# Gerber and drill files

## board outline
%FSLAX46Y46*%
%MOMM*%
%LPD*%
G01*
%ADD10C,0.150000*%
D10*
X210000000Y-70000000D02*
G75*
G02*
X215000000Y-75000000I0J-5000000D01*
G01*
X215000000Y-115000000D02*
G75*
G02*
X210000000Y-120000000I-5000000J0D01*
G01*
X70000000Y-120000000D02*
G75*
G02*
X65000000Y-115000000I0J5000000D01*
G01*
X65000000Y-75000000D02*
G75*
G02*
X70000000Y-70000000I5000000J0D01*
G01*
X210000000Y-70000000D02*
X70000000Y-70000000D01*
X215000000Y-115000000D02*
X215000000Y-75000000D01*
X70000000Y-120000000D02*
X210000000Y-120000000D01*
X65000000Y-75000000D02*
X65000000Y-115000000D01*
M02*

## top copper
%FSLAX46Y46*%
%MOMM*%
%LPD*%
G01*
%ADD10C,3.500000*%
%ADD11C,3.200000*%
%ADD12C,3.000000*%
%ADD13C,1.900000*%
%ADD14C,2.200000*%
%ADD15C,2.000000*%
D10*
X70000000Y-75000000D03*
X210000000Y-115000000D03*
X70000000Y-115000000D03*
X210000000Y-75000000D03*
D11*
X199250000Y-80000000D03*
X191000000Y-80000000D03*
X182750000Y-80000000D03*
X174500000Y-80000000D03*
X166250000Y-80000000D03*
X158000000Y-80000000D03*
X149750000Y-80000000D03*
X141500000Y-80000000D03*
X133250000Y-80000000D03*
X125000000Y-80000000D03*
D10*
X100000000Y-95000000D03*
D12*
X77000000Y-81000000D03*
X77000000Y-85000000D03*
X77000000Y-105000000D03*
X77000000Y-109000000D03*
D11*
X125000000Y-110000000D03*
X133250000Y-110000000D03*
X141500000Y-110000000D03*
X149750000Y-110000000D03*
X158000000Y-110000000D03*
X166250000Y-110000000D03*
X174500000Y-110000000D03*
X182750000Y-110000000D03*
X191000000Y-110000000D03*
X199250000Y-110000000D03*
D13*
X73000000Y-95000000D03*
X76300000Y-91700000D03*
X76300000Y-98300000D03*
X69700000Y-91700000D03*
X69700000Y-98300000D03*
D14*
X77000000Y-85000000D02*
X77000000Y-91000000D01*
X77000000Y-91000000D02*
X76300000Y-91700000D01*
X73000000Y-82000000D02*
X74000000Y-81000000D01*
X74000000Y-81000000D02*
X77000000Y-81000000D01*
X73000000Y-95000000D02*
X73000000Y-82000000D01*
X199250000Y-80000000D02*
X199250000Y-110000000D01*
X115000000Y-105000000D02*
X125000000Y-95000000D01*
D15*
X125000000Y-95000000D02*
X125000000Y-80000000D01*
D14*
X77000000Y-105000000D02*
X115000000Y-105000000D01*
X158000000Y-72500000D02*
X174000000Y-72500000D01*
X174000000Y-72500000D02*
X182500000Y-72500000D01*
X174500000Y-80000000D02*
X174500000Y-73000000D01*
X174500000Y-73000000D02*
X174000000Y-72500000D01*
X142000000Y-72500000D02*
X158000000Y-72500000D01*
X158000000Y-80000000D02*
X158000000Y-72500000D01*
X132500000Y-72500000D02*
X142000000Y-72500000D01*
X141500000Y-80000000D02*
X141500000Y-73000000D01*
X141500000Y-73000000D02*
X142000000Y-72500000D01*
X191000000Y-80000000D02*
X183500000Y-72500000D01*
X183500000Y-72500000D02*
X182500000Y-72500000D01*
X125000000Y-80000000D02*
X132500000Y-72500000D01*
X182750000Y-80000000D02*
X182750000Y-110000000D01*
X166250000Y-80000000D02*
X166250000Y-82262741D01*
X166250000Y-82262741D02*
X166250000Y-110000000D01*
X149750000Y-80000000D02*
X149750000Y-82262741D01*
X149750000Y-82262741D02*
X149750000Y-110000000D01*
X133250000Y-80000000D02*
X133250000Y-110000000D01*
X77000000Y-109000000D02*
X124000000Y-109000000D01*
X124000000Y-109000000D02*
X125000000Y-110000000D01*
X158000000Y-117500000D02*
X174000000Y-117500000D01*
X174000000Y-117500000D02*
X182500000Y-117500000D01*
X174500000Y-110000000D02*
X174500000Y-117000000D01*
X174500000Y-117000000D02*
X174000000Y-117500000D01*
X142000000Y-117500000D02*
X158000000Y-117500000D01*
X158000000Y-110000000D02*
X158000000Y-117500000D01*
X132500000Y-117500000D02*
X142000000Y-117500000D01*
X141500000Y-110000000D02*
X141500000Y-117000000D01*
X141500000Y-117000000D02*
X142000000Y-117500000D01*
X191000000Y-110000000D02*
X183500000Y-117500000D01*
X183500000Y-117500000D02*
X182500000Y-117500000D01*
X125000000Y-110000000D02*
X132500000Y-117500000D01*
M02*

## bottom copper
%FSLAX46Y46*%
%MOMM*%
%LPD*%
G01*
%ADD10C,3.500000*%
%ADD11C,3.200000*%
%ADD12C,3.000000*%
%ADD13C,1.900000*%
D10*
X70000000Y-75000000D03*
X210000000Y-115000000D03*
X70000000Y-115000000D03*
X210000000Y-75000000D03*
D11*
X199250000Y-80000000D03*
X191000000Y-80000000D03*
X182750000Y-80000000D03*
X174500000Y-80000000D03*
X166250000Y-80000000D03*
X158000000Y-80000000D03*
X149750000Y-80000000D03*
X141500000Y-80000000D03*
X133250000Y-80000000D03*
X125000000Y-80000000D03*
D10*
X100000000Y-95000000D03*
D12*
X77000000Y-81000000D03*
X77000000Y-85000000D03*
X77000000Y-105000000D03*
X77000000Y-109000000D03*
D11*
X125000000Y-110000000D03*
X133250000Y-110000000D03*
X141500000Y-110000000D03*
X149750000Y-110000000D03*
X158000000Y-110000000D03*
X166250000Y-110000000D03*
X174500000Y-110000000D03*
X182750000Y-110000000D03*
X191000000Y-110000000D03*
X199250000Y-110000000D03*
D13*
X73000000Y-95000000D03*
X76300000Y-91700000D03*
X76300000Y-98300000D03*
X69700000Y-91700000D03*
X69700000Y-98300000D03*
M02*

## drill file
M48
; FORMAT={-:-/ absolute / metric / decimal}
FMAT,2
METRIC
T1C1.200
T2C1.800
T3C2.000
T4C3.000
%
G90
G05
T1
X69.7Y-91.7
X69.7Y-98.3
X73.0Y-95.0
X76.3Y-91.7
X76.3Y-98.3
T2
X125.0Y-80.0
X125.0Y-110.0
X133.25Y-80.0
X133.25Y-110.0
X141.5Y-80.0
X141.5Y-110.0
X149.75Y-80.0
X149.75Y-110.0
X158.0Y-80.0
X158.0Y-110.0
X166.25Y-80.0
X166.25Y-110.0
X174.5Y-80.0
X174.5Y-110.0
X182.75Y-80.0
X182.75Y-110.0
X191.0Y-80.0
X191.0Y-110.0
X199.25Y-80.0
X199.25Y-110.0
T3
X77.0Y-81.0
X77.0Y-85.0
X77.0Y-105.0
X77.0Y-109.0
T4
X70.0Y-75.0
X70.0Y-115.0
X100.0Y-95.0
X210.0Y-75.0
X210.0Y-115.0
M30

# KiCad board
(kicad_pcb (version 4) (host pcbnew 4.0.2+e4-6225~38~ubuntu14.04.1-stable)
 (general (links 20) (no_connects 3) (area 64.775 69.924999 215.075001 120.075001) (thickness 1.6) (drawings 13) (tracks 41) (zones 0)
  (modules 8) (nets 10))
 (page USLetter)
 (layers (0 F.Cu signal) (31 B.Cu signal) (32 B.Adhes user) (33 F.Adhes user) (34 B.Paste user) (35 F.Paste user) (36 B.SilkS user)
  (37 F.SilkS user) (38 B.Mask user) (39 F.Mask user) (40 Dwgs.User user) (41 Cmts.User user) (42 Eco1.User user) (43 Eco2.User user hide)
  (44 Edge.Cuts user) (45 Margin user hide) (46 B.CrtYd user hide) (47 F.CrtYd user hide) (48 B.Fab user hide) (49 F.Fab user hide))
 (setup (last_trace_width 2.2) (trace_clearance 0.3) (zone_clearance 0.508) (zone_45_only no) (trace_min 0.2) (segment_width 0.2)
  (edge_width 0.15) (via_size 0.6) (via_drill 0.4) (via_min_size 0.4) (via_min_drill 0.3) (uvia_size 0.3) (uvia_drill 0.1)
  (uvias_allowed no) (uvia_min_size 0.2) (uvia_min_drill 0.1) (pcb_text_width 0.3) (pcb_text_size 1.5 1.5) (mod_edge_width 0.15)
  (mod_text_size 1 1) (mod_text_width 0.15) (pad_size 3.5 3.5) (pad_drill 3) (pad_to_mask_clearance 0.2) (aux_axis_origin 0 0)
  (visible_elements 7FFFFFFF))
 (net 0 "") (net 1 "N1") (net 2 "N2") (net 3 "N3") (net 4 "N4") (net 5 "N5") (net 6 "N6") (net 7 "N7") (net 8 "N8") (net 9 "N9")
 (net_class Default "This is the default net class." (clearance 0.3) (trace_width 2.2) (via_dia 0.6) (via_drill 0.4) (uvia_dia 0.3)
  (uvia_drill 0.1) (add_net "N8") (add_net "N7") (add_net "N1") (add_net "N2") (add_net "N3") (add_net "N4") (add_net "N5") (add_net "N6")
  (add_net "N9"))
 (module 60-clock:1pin (layer F.Cu) (at 70 75)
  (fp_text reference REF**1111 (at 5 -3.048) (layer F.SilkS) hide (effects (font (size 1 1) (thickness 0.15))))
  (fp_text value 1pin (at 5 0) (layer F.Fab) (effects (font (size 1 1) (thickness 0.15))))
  (pad 1 thru_hole circle (at 0 0) (size 3.5 3.5) (drill 3) (layers *.Cu *.Mask)))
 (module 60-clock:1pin (layer F.Cu) (at 210 115)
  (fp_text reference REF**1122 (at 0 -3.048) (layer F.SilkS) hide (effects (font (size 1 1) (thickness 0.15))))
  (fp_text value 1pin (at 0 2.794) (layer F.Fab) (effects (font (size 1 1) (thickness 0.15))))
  (pad 1 thru_hole circle (at 0 0) (size 3.5 3.5) (drill 3) (layers *.Cu *.Mask)))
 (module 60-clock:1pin (layer F.Cu) (at 70 115)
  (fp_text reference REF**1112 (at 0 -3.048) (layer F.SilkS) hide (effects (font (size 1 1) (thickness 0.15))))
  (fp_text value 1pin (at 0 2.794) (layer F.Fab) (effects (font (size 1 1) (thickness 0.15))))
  (pad 1 thru_hole circle (at 0 0) (size 3.5 3.5) (drill 3) (layers *.Cu *.Mask)))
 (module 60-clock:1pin (layer F.Cu) (at 210 75)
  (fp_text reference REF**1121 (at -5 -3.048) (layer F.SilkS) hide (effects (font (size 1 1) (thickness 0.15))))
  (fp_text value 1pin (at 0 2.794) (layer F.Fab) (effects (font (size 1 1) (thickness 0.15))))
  (pad 1 thru_hole circle (at 0 0) (size 3.5 3.5) (drill 3) (layers *.Cu *.Mask)))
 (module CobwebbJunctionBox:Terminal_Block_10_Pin (layer F.Cu) (at 199.25 80 180)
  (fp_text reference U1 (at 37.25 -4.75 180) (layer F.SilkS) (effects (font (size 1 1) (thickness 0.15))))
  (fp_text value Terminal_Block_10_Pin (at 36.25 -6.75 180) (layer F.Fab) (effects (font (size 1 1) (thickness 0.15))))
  (pad 1 thru_hole circle (at 0 0 180) (size 3.2 3.2) (drill 1.8) (layers *.Cu *.Mask F.SilkS) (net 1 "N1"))
  (pad 2 thru_hole circle (at 8.25 0 180) (size 3.2 3.2) (drill 1.8) (layers *.Cu *.Mask F.SilkS) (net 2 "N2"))
  (pad 3 thru_hole circle (at 16.5 0 180) (size 3.2 3.2) (drill 1.8) (layers *.Cu *.Mask F.SilkS) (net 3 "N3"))
  (pad 4 thru_hole circle (at 24.75 0 180) (size 3.2 3.2) (drill 1.8) (layers *.Cu *.Mask F.SilkS) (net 2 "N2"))
  (pad 5 thru_hole circle (at 33 0 180) (size 3.2 3.2) (drill 1.8) (layers *.Cu *.Mask F.SilkS) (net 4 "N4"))
  (pad 6 thru_hole circle (at 41.25 0 180) (size 3.2 3.2) (drill 1.8) (layers *.Cu *.Mask F.SilkS) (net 2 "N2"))
  (pad 7 thru_hole circle (at 49.5 0 180) (size 3.2 3.2) (drill 1.8) (layers *.Cu *.Mask F.SilkS) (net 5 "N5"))
  (pad 8 thru_hole circle (at 57.75 0 180) (size 3.2 3.2) (drill 1.8) (layers *.Cu *.Mask F.SilkS) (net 2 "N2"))
  (pad 9 thru_hole circle (at 66 0 180) (size 3.2 3.2) (drill 1.8) (layers *.Cu *.Mask F.SilkS) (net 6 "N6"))
  (pad 10 thru_hole circle (at 74.25 0 180) (size 3.2 3.2) (drill 1.8) (layers *.Cu *.Mask F.SilkS) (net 2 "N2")))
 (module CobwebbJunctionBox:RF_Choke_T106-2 (layer F.Cu) (at 100 95)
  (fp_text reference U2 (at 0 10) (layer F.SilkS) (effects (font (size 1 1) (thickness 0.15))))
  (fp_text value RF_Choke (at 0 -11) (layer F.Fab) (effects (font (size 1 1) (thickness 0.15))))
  (pad "" thru_hole circle (at 0 0) (size 3.5 3.5) (drill 3) (layers *.Cu *.Mask F.SilkS))
  (pad 1 thru_hole circle (at -23 -14) (size 3 3) (drill 2) (layers *.Cu *.Mask F.SilkS) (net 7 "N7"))
  (pad 2 thru_hole circle (at -23 -10) (size 3 3) (drill 2) (layers *.Cu *.Mask F.SilkS) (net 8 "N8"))
  (pad 3 thru_hole circle (at -23 10) (size 3 3) (drill 2) (layers *.Cu *.Mask F.SilkS) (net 2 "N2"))
  (pad 4 thru_hole circle (at -23 14) (size 3 3) (drill 2) (layers *.Cu *.Mask F.SilkS) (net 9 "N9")))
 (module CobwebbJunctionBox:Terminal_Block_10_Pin (layer F.Cu) (at 125 110)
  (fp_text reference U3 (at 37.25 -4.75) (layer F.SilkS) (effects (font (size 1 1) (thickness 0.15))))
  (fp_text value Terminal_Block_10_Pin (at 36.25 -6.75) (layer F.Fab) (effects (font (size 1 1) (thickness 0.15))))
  (pad 1 thru_hole circle (at 0 0) (size 3.2 3.2) (drill 1.8) (layers *.Cu *.Mask F.SilkS) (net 9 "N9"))
  (pad 2 thru_hole circle (at 8.25 0) (size 3.2 3.2) (drill 1.8) (layers *.Cu *.Mask F.SilkS) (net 6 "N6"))
  (pad 3 thru_hole circle (at 16.5 0) (size 3.2 3.2) (drill 1.8) (layers *.Cu *.Mask F.SilkS) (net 9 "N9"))
  (pad 4 thru_hole circle (at 24.75 0) (size 3.2 3.2) (drill 1.8) (layers *.Cu *.Mask F.SilkS) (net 5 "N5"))
  (pad 5 thru_hole circle (at 33 0) (size 3.2 3.2) (drill 1.8) (layers *.Cu *.Mask F.SilkS) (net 9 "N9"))
  (pad 6 thru_hole circle (at 41.25 0) (size 3.2 3.2) (drill 1.8) (layers *.Cu *.Mask F.SilkS) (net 4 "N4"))
  (pad 7 thru_hole circle (at 49.5 0) (size 3.2 3.2) (drill 1.8) (layers *.Cu *.Mask F.SilkS) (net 9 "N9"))
  (pad 8 thru_hole circle (at 57.75 0) (size 3.2 3.2) (drill 1.8) (layers *.Cu *.Mask F.SilkS) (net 3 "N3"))
  (pad 9 thru_hole circle (at 66 0) (size 3.2 3.2) (drill 1.8) (layers *.Cu *.Mask F.SilkS) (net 9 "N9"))
  (pad 10 thru_hole circle (at 74.25 0) (size 3.2 3.2) (drill 1.8) (layers *.Cu *.Mask F.SilkS) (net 1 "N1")))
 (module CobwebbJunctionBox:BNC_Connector (layer F.Cu) (at 73 95 270)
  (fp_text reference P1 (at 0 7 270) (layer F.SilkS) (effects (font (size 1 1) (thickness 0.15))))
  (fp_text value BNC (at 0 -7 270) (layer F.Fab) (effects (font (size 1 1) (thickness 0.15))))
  (pad 2 thru_hole circle (at 0 0 270) (size 1.9 1.9) (drill 1.2) (layers *.Cu *.Mask F.SilkS) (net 7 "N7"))
  (pad 1 thru_hole circle (at -3.3 -3.3 270) (size 1.9 1.9) (drill 1.2) (layers *.Cu *.Mask F.SilkS) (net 8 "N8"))
  (pad 1 thru_hole circle (at 3.3 -3.3 270) (size 1.9 1.9) (drill 1.2) (layers *.Cu *.Mask F.SilkS) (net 8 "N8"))
  (pad 1 thru_hole circle (at -3.3 3.3 270) (size 1.9 1.9) (drill 1.2) (layers *.Cu *.Mask F.SilkS) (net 8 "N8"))
  (pad 1 thru_hole circle (at 3.3 3.3 270) (size 1.9 1.9) (drill 1.2) (layers *.Cu *.Mask F.SilkS) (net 8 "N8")))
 (gr_arc (start 210 75) (end 210 70) (angle 90) (layer Edge.Cuts) (width 0.15))
 (gr_arc (start 210 115) (end 215 115) (angle 90) (layer Edge.Cuts) (width 0.15))
 (gr_arc (start 70 115) (end 70 120) (angle 90) (layer Edge.Cuts) (width 0.15))
 (gr_arc (start 70 75) (end 65 75) (angle 90) (layer Edge.Cuts) (width 0.15))
 (gr_line (start 210 70) (end 70 70) (layer Edge.Cuts) (width 0.15))
 (gr_line (start 215 115) (end 215 75) (layer Edge.Cuts) (width 0.15))
 (gr_line (start 70 120) (end 210 120) (layer Edge.Cuts) (width 0.15))
 (gr_line (start 65 75) (end 65 115) (layer Edge.Cuts) (width 0.15))
 (segment (start 77 85) (end 77 91) (width 2.2) (layer F.Cu) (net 8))
 (segment (start 77 91) (end 76.3 91.7) (width 2.2) (layer F.Cu) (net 8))
 (segment (start 73 82) (end 74 81) (width 2.2) (layer F.Cu) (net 7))
 (segment (start 74 81) (end 77 81) (width 2.2) (layer F.Cu) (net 7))
 (segment (start 73 95) (end 73 82) (width 2.2) (layer F.Cu) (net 7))
 (segment (start 199.25 80) (end 199.25 110) (width 2.2) (layer F.Cu) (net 1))
 (segment (start 115 105) (end 125 95) (width 2.2) (layer F.Cu) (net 2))
 (segment (start 125 95) (end 125 80) (width 2) (layer F.Cu) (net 2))
 (segment (start 77 105) (end 115 105) (width 2.2) (layer F.Cu) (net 2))
 (segment (start 158 72.5) (end 174 72.5) (width 2.2) (layer F.Cu) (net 2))
 (segment (start 174 72.5) (end 182.5 72.5) (width 2.2) (layer F.Cu) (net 2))
 (segment (start 174.5 80) (end 174.5 73) (width 2.2) (layer F.Cu) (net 2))
 (segment (start 174.5 73) (end 174 72.5) (width 2.2) (layer F.Cu) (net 2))
 (segment (start 142 72.5) (end 158 72.5) (width 2.2) (layer F.Cu) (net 2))
 (segment (start 158 80) (end 158 72.5) (width 2.2) (layer F.Cu) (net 2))
 (segment (start 132.5 72.5) (end 142 72.5) (width 2.2) (layer F.Cu) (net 2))
 (segment (start 141.5 80) (end 141.5 73) (width 2.2) (layer F.Cu) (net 2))
 (segment (start 141.5 73) (end 142 72.5) (width 2.2) (layer F.Cu) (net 2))
 (segment (start 191 80) (end 183.5 72.5) (width 2.2) (layer F.Cu) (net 2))
 (segment (start 183.5 72.5) (end 182.5 72.5) (width 2.2) (layer F.Cu) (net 2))
 (segment (start 125 80) (end 132.5 72.5) (width 2.2) (layer F.Cu) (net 2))
 (segment (start 182.75 80) (end 182.75 110) (width 2.2) (layer F.Cu) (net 3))
 (segment (start 166.25 80) (end 166.25 82.262741) (width 2.2) (layer F.Cu) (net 4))
 (segment (start 166.25 82.262741) (end 166.25 110) (width 2.2) (layer F.Cu) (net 4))
 (segment (start 149.75 80) (end 149.75 82.262741) (width 2.2) (layer F.Cu) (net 5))
 (segment (start 149.75 82.262741) (end 149.75 110) (width 2.2) (layer F.Cu) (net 5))
 (segment (start 133.25 80) (end 133.25 110) (width 2.2) (layer F.Cu) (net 6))
 (segment (start 77 109) (end 124 109) (width 2.2) (layer F.Cu) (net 9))
 (segment (start 124 109) (end 125 110) (width 2.2) (layer F.Cu) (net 9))
 (segment (start 158 117.5) (end 174 117.5) (width 2.2) (layer F.Cu) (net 9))
 (segment (start 174 117.5) (end 182.5 117.5) (width 2.2) (layer F.Cu) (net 9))
 (segment (start 174.5 110) (end 174.5 117) (width 2.2) (layer F.Cu) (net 9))
 (segment (start 174.5 117) (end 174 117.5) (width 2.2) (layer F.Cu) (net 9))
 (segment (start 142 117.5) (end 158 117.5) (width 2.2) (layer F.Cu) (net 9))
 (segment (start 158 110) (end 158 117.5) (width 2.2) (layer F.Cu) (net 9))
 (segment (start 132.5 117.5) (end 142 117.5) (width 2.2) (layer F.Cu) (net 9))
 (segment (start 141.5 110) (end 141.5 117) (width 2.2) (layer F.Cu) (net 9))
 (segment (start 141.5 117) (end 142 117.5) (width 2.2) (layer F.Cu) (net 9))
 (segment (start 191 110) (end 183.5 117.5) (width 2.2) (layer F.Cu) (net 9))
 (segment (start 183.5 117.5) (end 182.5 117.5) (width 2.2) (layer F.Cu) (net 9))
 (segment (start 125 110) (end 132.5 117.5) (width 2.2) (layer F.Cu) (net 9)))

